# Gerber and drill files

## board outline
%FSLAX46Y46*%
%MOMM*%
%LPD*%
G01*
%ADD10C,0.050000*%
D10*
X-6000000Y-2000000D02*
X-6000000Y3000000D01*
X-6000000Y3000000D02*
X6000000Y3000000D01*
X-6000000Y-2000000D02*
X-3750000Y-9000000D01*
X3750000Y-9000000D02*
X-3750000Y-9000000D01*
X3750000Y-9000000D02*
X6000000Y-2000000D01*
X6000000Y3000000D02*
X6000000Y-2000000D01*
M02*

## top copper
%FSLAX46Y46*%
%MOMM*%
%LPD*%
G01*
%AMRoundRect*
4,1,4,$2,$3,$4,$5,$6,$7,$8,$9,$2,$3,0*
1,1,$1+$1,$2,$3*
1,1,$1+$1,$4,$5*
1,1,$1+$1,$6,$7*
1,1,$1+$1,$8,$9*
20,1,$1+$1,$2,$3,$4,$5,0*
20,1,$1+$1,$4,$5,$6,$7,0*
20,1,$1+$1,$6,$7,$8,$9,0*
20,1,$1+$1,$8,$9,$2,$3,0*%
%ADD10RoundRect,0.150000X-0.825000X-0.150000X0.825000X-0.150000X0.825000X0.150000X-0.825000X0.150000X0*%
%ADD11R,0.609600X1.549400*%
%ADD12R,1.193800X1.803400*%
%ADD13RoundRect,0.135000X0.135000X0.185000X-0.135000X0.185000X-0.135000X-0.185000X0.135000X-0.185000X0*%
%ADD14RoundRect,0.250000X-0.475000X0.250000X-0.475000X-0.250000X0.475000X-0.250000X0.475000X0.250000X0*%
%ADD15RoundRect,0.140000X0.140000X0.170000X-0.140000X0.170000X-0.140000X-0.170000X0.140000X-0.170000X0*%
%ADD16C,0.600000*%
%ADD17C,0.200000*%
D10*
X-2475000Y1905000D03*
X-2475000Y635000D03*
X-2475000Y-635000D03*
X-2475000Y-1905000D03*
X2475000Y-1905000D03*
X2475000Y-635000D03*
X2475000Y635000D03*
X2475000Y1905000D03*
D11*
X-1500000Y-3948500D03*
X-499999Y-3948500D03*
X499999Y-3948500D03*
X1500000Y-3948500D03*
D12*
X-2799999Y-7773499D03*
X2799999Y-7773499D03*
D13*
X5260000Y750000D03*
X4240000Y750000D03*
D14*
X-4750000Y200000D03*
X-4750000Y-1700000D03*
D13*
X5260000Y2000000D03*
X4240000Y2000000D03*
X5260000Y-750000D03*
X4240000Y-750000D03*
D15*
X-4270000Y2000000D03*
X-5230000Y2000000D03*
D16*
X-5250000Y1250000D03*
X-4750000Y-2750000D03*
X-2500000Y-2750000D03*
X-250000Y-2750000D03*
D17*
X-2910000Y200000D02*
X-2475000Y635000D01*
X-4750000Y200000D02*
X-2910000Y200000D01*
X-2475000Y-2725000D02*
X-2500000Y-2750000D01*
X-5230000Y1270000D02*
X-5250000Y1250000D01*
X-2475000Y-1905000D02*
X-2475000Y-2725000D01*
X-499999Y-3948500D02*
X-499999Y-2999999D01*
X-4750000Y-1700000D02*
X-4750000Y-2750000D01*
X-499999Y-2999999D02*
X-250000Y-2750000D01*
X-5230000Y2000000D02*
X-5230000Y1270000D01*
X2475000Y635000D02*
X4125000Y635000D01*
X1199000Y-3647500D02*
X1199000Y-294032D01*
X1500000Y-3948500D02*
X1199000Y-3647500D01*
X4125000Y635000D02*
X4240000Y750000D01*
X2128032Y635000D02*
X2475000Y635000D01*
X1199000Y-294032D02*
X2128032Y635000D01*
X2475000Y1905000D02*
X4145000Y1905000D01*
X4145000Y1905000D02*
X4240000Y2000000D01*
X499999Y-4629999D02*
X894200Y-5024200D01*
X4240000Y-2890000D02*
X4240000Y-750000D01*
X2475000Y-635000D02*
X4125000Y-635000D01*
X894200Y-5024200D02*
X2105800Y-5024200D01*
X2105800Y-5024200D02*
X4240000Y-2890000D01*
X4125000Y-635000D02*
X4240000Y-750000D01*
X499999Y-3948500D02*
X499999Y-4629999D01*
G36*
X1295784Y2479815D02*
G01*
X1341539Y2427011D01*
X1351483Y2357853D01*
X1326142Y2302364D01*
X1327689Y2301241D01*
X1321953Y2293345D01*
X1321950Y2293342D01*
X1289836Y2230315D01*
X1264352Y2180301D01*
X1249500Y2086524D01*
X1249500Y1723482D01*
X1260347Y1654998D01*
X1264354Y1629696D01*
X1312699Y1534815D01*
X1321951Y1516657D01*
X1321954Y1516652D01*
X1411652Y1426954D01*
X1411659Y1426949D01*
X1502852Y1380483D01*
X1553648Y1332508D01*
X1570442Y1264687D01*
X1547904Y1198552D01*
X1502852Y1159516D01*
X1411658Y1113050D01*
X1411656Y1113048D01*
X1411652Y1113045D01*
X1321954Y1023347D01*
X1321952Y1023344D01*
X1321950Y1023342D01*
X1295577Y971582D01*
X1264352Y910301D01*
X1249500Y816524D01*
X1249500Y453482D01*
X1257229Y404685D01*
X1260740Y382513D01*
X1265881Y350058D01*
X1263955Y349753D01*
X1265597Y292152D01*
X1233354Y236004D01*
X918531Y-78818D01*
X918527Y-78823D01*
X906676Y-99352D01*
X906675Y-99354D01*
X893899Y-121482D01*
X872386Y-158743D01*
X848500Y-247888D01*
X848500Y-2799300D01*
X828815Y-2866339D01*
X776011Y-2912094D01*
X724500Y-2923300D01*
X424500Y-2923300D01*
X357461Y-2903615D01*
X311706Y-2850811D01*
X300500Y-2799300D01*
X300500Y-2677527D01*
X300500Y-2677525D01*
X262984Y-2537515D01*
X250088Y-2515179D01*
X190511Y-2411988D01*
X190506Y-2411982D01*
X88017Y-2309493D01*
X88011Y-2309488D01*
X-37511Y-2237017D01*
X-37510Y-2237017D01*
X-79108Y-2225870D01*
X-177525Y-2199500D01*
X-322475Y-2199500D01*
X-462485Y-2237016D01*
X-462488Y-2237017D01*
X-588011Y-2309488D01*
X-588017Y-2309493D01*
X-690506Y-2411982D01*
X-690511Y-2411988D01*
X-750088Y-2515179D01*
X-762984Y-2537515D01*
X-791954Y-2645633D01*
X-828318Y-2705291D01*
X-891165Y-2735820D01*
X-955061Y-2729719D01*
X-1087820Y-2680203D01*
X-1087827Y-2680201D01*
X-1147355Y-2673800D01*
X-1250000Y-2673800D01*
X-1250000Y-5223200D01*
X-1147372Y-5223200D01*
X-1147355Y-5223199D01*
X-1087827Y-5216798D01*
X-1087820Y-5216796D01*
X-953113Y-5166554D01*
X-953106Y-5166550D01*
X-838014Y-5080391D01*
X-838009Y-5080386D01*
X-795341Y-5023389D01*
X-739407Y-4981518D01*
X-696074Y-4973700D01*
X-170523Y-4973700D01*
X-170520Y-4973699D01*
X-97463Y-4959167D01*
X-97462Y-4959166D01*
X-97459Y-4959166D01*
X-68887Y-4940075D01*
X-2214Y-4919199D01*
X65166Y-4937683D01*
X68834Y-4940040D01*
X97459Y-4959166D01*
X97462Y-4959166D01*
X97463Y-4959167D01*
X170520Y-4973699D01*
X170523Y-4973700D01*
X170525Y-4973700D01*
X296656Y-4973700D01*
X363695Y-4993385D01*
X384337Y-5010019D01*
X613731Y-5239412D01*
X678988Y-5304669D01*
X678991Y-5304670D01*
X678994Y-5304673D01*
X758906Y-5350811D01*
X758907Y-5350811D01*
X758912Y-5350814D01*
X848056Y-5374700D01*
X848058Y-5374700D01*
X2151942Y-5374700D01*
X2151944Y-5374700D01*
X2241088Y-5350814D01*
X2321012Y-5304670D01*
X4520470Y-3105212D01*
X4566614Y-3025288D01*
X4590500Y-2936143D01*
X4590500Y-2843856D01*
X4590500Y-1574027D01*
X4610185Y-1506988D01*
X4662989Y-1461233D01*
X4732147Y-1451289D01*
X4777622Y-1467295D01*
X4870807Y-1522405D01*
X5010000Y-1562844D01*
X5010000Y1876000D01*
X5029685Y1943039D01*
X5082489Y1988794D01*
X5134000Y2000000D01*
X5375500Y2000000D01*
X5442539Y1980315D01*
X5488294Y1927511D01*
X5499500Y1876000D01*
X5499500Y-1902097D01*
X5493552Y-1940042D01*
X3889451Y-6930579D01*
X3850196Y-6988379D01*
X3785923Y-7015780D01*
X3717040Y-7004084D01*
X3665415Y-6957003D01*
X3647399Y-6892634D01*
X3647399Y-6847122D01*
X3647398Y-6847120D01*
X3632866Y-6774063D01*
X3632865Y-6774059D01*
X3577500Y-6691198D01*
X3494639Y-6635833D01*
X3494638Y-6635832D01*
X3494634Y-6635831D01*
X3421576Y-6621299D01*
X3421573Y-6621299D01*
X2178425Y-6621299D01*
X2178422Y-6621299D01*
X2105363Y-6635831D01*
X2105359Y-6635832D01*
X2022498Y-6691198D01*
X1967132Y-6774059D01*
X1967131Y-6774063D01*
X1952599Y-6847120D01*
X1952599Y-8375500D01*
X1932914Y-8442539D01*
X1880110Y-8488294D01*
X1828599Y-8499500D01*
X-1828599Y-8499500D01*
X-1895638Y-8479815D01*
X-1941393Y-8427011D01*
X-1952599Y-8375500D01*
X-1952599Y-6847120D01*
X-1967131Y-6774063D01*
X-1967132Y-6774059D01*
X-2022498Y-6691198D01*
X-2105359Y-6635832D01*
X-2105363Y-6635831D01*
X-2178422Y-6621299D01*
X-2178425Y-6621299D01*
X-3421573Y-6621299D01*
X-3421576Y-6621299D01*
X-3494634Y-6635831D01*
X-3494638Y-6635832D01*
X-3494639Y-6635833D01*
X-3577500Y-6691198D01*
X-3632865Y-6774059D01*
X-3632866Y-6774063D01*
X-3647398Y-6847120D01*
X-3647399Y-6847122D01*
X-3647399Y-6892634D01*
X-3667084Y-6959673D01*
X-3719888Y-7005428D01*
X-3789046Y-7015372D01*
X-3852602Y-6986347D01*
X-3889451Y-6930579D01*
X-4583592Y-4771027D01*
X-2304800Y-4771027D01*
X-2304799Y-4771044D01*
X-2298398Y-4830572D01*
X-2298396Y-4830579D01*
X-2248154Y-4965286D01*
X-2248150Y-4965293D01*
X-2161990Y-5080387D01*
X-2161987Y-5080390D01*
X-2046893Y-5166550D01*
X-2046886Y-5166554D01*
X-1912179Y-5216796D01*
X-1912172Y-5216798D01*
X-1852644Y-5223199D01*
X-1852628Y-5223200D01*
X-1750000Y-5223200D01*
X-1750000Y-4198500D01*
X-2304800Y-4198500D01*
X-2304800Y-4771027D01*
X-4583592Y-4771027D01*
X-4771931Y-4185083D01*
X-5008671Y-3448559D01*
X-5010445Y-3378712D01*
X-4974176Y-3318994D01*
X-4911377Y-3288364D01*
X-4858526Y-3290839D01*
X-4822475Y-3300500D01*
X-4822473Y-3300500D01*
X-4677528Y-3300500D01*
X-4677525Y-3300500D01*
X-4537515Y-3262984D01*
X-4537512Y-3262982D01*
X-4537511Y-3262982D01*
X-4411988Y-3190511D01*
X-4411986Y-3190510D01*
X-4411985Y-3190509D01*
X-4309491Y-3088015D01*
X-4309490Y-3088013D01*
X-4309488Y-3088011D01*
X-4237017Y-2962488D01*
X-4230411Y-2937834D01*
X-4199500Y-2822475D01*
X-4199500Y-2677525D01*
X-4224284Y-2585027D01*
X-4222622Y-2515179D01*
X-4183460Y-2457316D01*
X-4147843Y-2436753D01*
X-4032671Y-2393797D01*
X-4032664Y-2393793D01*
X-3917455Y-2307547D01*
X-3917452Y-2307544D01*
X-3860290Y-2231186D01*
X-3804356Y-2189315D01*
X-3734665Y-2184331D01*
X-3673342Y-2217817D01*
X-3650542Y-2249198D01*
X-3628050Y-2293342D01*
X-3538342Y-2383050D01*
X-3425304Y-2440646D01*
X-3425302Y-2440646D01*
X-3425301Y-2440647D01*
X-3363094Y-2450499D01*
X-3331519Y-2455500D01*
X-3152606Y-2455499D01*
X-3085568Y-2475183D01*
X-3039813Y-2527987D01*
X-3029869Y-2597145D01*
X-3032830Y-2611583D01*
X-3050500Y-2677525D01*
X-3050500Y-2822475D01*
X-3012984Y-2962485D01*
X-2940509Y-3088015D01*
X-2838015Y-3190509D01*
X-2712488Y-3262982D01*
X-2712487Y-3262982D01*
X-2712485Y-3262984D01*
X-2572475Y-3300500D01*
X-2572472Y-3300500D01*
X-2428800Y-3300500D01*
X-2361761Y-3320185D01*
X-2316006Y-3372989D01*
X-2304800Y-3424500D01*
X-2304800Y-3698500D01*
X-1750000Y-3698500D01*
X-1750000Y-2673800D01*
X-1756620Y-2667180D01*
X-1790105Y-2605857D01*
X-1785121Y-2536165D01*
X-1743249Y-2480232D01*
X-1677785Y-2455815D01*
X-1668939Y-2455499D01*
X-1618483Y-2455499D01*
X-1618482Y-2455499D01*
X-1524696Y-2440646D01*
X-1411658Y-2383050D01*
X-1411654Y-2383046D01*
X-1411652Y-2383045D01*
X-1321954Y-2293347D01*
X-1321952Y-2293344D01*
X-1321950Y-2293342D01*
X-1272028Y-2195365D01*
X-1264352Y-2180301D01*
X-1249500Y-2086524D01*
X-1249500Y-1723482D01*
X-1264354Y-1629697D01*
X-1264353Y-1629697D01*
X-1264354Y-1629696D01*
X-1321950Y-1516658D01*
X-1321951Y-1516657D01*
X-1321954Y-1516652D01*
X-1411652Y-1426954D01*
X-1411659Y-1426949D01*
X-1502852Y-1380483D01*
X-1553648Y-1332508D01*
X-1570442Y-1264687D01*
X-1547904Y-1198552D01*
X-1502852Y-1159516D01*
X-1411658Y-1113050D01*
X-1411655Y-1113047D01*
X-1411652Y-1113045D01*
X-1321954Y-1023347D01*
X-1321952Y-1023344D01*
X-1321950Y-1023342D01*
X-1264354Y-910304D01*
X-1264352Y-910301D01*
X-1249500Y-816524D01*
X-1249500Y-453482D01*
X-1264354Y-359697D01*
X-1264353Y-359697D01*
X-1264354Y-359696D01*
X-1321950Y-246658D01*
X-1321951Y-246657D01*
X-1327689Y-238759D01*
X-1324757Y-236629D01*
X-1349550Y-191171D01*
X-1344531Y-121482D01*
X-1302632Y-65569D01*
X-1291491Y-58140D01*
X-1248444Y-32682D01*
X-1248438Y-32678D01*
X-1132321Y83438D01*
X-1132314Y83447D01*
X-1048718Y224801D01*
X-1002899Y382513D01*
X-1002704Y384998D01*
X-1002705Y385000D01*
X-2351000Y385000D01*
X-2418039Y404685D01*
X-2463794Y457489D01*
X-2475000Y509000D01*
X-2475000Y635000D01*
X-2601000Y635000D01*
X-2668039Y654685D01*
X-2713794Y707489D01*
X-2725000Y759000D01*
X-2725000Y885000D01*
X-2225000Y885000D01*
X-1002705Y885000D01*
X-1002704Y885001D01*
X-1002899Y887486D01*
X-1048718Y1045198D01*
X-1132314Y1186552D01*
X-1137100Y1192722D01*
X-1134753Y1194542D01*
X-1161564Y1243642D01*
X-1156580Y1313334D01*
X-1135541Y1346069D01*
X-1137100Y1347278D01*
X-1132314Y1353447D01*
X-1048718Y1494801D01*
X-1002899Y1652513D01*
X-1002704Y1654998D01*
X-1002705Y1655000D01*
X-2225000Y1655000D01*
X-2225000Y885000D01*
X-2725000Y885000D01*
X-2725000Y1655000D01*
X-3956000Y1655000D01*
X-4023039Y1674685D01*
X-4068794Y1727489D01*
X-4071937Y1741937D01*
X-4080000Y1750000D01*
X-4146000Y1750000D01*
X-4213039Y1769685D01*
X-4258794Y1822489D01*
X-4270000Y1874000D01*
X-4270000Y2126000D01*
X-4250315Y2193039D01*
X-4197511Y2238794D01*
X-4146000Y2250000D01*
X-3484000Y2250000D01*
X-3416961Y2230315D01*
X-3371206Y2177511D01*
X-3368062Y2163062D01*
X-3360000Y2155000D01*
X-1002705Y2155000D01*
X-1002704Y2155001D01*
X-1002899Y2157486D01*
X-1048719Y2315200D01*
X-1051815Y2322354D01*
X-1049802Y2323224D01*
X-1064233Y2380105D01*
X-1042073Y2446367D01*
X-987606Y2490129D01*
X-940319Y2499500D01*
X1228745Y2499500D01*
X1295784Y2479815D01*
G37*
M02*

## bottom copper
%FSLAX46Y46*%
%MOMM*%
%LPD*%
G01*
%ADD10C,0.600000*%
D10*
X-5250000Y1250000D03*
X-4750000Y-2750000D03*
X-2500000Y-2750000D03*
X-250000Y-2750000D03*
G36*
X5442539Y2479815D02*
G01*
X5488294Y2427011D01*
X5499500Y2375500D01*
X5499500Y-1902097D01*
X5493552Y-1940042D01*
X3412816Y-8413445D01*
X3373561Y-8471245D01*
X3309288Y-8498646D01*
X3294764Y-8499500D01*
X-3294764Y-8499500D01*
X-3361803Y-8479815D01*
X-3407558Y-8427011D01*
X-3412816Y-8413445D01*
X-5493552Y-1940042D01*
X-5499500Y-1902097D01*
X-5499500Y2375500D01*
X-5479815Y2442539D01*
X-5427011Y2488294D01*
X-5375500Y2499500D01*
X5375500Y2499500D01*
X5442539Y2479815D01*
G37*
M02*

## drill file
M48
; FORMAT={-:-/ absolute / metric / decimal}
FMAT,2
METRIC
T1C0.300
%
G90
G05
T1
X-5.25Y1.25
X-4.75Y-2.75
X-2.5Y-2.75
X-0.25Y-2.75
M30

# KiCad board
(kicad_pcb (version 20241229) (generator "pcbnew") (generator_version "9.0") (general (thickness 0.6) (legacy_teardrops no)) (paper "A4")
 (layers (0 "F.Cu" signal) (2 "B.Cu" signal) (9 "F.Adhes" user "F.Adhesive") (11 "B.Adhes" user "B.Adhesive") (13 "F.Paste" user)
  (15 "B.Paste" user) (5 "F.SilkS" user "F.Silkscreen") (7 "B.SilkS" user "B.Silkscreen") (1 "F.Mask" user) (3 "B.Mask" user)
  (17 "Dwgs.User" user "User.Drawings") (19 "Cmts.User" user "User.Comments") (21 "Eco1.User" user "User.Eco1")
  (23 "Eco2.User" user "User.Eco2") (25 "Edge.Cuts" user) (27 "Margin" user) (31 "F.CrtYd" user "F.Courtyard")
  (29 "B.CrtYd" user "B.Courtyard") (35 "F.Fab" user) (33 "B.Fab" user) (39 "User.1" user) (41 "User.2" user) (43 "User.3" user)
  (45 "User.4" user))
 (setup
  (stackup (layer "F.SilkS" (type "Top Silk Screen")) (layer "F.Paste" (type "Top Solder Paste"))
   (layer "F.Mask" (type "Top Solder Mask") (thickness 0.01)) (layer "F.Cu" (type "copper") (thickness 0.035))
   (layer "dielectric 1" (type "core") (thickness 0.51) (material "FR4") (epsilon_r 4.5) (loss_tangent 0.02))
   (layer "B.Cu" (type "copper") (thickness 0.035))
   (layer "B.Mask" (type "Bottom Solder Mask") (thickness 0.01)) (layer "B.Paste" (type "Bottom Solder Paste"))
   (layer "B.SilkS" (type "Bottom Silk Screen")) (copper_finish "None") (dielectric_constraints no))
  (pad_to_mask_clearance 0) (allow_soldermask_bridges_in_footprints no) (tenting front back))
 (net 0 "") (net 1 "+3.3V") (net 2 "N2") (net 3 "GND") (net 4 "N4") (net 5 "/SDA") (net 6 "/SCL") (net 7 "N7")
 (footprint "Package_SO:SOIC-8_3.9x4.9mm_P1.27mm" (layer "F.Cu") (at 0 0)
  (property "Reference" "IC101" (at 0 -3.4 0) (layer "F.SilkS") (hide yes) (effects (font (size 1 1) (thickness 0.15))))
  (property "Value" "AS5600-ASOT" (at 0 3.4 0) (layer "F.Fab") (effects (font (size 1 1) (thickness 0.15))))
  (pad "1" smd roundrect (at -2.475 -1.905) (size 1.95 0.6) (layers "F.Cu" "F.Mask" "F.Paste") (roundrect_rratio 0.25) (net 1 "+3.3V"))
  (pad "2" smd roundrect (at -2.475 -0.635) (size 1.95 0.6) (layers "F.Cu" "F.Mask" "F.Paste") (roundrect_rratio 0.25) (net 1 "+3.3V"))
  (pad "3" smd roundrect (at -2.475 0.635) (size 1.95 0.6) (layers "F.Cu" "F.Mask" "F.Paste") (roundrect_rratio 0.25) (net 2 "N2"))
  (pad "4" smd roundrect (at -2.475 1.905) (size 1.95 0.6) (layers "F.Cu" "F.Mask" "F.Paste") (roundrect_rratio 0.25) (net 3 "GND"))
  (pad "5" smd roundrect (at 2.475 1.905) (size 1.95 0.6) (layers "F.Cu" "F.Mask" "F.Paste") (roundrect_rratio 0.25) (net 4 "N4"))
  (pad "6" smd roundrect (at 2.475 0.635) (size 1.95 0.6) (layers "F.Cu" "F.Mask" "F.Paste") (roundrect_rratio 0.25) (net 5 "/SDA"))
  (pad "7" smd roundrect (at 2.475 -0.635) (size 1.95 0.6) (layers "F.Cu" "F.Mask" "F.Paste") (roundrect_rratio 0.25) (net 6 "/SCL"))
  (pad "8" smd roundrect (at 2.475 -1.905) (size 1.95 0.6) (layers "F.Cu" "F.Mask" "F.Paste") (roundrect_rratio 0.25) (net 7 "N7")))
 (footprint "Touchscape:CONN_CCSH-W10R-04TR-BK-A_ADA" (layer "F.Cu") (at 0 6)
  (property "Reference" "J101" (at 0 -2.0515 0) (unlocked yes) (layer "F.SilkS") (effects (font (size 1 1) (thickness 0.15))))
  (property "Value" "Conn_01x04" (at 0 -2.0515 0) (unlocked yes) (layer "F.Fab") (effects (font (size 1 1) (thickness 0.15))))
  (pad "1" smd rect (at -1.5 -2.0515) (size 0.6096 1.5494) (layers "F.Cu" "F.Mask" "F.Paste") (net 1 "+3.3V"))
  (pad "2" smd rect (at -0.499999 -2.0515) (size 0.6096 1.5494) (layers "F.Cu" "F.Mask" "F.Paste") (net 3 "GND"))
  (pad "3" smd rect (at 0.499999 -2.0515) (size 0.6096 1.5494) (layers "F.Cu" "F.Mask" "F.Paste") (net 5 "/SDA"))
  (pad "4" smd rect (at 1.5 -2.0515) (size 0.6096 1.5494) (layers "F.Cu" "F.Mask" "F.Paste") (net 6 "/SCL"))
  (pad "5" smd rect (at -2.799999 1.773499) (size 1.1938 1.8034) (layers "F.Cu" "F.Mask" "F.Paste"))
  (pad "6" smd rect (at 2.799999 1.773499) (size 1.1938 1.8034) (layers "F.Cu" "F.Mask" "F.Paste")))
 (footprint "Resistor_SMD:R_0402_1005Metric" (layer "F.Cu") (at 4.75 -0.75 180)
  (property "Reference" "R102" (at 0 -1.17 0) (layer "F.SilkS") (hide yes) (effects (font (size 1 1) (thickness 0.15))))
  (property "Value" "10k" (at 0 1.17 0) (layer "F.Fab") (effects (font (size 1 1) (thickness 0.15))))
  (pad "1" smd roundrect (at -0.51 0 180) (size 0.54 0.64) (layers "F.Cu" "F.Mask" "F.Paste") (roundrect_rratio 0.25) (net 1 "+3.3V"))
  (pad "2" smd roundrect (at 0.51 0 180) (size 0.54 0.64) (layers "F.Cu" "F.Mask" "F.Paste") (roundrect_rratio 0.25) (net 6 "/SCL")))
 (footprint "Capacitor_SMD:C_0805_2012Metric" (layer "F.Cu") (at -4.75 0.75 -90)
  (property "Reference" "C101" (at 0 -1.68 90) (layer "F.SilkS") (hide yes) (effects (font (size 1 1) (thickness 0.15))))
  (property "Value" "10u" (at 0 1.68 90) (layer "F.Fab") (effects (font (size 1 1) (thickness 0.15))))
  (pad "1" smd roundrect (at -0.95 0 270) (size 1 1.45) (layers "F.Cu" "F.Mask" "F.Paste") (roundrect_rratio 0.25) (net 1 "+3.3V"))
  (pad "2" smd roundrect (at 0.95 0 270) (size 1 1.45) (layers "F.Cu" "F.Mask" "F.Paste") (roundrect_rratio 0.25) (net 3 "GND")))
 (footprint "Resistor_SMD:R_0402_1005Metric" (layer "F.Cu") (at 4.75 -2 180)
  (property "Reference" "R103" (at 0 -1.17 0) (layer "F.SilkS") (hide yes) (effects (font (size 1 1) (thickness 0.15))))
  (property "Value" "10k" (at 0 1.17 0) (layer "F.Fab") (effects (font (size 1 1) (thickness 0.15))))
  (pad "1" smd roundrect (at -0.51 0 180) (size 0.54 0.64) (layers "F.Cu" "F.Mask" "F.Paste") (roundrect_rratio 0.25) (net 1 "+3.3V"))
  (pad "2" smd roundrect (at 0.51 0 180) (size 0.54 0.64) (layers "F.Cu" "F.Mask" "F.Paste") (roundrect_rratio 0.25) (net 7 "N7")))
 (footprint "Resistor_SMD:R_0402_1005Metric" (layer "F.Cu") (at 4.75 0.75 180)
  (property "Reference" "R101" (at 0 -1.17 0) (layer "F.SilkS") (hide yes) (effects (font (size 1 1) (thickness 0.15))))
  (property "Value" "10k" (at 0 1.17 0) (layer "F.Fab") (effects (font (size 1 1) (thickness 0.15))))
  (pad "1" smd roundrect (at -0.51 0 180) (size 0.54 0.64) (layers "F.Cu" "F.Mask" "F.Paste") (roundrect_rratio 0.25) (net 1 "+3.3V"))
  (pad "2" smd roundrect (at 0.51 0 180) (size 0.54 0.64) (layers "F.Cu" "F.Mask" "F.Paste") (roundrect_rratio 0.25) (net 5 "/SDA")))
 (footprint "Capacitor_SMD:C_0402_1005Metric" (layer "F.Cu") (at -4.75 -2 180)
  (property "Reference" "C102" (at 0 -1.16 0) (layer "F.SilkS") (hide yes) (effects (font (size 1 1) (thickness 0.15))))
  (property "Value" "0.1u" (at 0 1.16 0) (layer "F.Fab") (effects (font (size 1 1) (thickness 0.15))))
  (pad "1" smd roundrect (at -0.48 0 180) (size 0.56 0.62) (layers "F.Cu" "F.Mask" "F.Paste") (roundrect_rratio 0.25) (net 1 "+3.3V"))
  (pad "2" smd roundrect (at 0.48 0 180) (size 0.56 0.62) (layers "F.Cu" "F.Mask" "F.Paste") (roundrect_rratio 0.25) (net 3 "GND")))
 (gr_line (start -6 2) (end -6 -3) (stroke (width 0.05) (type default)) (layer "Edge.Cuts"))
 (gr_line (start -6 -3) (end 6 -3) (stroke (width 0.05) (type default)) (layer "Edge.Cuts"))
 (gr_line (start -6 2) (end -3.75 9) (stroke (width 0.05) (type default)) (layer "Edge.Cuts"))
 (gr_line (start 3.75 9) (end -3.75 9) (stroke (width 0.05) (type default)) (layer "Edge.Cuts"))
 (gr_line (start 3.75 9) (end 6 2) (stroke (width 0.05) (type default)) (layer "Edge.Cuts"))
 (gr_line (start 6 -3) (end 6 2) (stroke (width 0.05) (type default)) (layer "Edge.Cuts"))
 (segment (start -2.91 -0.2) (end -2.475 -0.635) (width 0.2) (layer "F.Cu") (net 1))
 (segment (start -4.75 -0.2) (end -2.91 -0.2) (width 0.2) (layer "F.Cu") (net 1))
 (segment (start -2.475 2.725) (end -2.5 2.75) (width 0.2) (layer "F.Cu") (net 3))
 (segment (start -5.23 -1.27) (end -5.25 -1.25) (width 0.2) (layer "F.Cu") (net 3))
 (segment (start -2.475 1.905) (end -2.475 2.725) (width 0.2) (layer "F.Cu") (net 3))
 (segment (start -0.499999 3.9485) (end -0.499999 2.999999) (width 0.2) (layer "F.Cu") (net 3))
 (segment (start -4.75 1.7) (end -4.75 2.75) (width 0.2) (layer "F.Cu") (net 3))
 (segment (start -0.499999 2.999999) (end -0.25 2.75) (width 0.2) (layer "F.Cu") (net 3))
 (segment (start -5.23 -2) (end -5.23 -1.27) (width 0.2) (layer "F.Cu") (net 3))
 (via (at -5.25 -1.25) (size 0.6) (drill 0.3) (layers "F.Cu" "B.Cu") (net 3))
 (via (at -4.75 2.75) (size 0.6) (drill 0.3) (layers "F.Cu" "B.Cu") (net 3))
 (via (at -2.5 2.75) (size 0.6) (drill 0.3) (layers "F.Cu" "B.Cu") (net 3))
 (via (at -0.25 2.75) (size 0.6) (drill 0.3) (layers "F.Cu" "B.Cu") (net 3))
 (segment (start 2.475 -0.635) (end 4.125 -0.635) (width 0.2) (layer "F.Cu") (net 6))
 (segment (start 1.199 3.6475) (end 1.199 0.294032) (width 0.2) (layer "F.Cu") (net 6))
 (segment (start 1.5 3.9485) (end 1.199 3.6475) (width 0.2) (layer "F.Cu") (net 6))
 (segment (start 4.125 -0.635) (end 4.24 -0.75) (width 0.2) (layer "F.Cu") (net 6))
 (segment (start 2.128032 -0.635) (end 2.475 -0.635) (width 0.2) (layer "F.Cu") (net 6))
 (segment (start 1.199 0.294032) (end 2.128032 -0.635) (width 0.2) (layer "F.Cu") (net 6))
 (segment (start 2.475 -1.905) (end 4.145 -1.905) (width 0.2) (layer "F.Cu") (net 7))
 (segment (start 4.145 -1.905) (end 4.24 -2) (width 0.2) (layer "F.Cu") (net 7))
 (segment (start 0.499999 4.629999) (end 0.8942 5.0242) (width 0.2) (layer "F.Cu") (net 5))
 (segment (start 4.24 2.89) (end 4.24 0.75) (width 0.2) (layer "F.Cu") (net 5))
 (segment (start 2.475 0.635) (end 4.125 0.635) (width 0.2) (layer "F.Cu") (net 5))
 (segment (start 0.8942 5.0242) (end 2.1058 5.0242) (width 0.2) (layer "F.Cu") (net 5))
 (segment (start 2.1058 5.0242) (end 4.24 2.89) (width 0.2) (layer "F.Cu") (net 5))
 (segment (start 4.125 0.635) (end 4.24 0.75) (width 0.2) (layer "F.Cu") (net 5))
 (segment (start 0.499999 3.9485) (end 0.499999 4.629999) (width 0.2) (layer "F.Cu") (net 5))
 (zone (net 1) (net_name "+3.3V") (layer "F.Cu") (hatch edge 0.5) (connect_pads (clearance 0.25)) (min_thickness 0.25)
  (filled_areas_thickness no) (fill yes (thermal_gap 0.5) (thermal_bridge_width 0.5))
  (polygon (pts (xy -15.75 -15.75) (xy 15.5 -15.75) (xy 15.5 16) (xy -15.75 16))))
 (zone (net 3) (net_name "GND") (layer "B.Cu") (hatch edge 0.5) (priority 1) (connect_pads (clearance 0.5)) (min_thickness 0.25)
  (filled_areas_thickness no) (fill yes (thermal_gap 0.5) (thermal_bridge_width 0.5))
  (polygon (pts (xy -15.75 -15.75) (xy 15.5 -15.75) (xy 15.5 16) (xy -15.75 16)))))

